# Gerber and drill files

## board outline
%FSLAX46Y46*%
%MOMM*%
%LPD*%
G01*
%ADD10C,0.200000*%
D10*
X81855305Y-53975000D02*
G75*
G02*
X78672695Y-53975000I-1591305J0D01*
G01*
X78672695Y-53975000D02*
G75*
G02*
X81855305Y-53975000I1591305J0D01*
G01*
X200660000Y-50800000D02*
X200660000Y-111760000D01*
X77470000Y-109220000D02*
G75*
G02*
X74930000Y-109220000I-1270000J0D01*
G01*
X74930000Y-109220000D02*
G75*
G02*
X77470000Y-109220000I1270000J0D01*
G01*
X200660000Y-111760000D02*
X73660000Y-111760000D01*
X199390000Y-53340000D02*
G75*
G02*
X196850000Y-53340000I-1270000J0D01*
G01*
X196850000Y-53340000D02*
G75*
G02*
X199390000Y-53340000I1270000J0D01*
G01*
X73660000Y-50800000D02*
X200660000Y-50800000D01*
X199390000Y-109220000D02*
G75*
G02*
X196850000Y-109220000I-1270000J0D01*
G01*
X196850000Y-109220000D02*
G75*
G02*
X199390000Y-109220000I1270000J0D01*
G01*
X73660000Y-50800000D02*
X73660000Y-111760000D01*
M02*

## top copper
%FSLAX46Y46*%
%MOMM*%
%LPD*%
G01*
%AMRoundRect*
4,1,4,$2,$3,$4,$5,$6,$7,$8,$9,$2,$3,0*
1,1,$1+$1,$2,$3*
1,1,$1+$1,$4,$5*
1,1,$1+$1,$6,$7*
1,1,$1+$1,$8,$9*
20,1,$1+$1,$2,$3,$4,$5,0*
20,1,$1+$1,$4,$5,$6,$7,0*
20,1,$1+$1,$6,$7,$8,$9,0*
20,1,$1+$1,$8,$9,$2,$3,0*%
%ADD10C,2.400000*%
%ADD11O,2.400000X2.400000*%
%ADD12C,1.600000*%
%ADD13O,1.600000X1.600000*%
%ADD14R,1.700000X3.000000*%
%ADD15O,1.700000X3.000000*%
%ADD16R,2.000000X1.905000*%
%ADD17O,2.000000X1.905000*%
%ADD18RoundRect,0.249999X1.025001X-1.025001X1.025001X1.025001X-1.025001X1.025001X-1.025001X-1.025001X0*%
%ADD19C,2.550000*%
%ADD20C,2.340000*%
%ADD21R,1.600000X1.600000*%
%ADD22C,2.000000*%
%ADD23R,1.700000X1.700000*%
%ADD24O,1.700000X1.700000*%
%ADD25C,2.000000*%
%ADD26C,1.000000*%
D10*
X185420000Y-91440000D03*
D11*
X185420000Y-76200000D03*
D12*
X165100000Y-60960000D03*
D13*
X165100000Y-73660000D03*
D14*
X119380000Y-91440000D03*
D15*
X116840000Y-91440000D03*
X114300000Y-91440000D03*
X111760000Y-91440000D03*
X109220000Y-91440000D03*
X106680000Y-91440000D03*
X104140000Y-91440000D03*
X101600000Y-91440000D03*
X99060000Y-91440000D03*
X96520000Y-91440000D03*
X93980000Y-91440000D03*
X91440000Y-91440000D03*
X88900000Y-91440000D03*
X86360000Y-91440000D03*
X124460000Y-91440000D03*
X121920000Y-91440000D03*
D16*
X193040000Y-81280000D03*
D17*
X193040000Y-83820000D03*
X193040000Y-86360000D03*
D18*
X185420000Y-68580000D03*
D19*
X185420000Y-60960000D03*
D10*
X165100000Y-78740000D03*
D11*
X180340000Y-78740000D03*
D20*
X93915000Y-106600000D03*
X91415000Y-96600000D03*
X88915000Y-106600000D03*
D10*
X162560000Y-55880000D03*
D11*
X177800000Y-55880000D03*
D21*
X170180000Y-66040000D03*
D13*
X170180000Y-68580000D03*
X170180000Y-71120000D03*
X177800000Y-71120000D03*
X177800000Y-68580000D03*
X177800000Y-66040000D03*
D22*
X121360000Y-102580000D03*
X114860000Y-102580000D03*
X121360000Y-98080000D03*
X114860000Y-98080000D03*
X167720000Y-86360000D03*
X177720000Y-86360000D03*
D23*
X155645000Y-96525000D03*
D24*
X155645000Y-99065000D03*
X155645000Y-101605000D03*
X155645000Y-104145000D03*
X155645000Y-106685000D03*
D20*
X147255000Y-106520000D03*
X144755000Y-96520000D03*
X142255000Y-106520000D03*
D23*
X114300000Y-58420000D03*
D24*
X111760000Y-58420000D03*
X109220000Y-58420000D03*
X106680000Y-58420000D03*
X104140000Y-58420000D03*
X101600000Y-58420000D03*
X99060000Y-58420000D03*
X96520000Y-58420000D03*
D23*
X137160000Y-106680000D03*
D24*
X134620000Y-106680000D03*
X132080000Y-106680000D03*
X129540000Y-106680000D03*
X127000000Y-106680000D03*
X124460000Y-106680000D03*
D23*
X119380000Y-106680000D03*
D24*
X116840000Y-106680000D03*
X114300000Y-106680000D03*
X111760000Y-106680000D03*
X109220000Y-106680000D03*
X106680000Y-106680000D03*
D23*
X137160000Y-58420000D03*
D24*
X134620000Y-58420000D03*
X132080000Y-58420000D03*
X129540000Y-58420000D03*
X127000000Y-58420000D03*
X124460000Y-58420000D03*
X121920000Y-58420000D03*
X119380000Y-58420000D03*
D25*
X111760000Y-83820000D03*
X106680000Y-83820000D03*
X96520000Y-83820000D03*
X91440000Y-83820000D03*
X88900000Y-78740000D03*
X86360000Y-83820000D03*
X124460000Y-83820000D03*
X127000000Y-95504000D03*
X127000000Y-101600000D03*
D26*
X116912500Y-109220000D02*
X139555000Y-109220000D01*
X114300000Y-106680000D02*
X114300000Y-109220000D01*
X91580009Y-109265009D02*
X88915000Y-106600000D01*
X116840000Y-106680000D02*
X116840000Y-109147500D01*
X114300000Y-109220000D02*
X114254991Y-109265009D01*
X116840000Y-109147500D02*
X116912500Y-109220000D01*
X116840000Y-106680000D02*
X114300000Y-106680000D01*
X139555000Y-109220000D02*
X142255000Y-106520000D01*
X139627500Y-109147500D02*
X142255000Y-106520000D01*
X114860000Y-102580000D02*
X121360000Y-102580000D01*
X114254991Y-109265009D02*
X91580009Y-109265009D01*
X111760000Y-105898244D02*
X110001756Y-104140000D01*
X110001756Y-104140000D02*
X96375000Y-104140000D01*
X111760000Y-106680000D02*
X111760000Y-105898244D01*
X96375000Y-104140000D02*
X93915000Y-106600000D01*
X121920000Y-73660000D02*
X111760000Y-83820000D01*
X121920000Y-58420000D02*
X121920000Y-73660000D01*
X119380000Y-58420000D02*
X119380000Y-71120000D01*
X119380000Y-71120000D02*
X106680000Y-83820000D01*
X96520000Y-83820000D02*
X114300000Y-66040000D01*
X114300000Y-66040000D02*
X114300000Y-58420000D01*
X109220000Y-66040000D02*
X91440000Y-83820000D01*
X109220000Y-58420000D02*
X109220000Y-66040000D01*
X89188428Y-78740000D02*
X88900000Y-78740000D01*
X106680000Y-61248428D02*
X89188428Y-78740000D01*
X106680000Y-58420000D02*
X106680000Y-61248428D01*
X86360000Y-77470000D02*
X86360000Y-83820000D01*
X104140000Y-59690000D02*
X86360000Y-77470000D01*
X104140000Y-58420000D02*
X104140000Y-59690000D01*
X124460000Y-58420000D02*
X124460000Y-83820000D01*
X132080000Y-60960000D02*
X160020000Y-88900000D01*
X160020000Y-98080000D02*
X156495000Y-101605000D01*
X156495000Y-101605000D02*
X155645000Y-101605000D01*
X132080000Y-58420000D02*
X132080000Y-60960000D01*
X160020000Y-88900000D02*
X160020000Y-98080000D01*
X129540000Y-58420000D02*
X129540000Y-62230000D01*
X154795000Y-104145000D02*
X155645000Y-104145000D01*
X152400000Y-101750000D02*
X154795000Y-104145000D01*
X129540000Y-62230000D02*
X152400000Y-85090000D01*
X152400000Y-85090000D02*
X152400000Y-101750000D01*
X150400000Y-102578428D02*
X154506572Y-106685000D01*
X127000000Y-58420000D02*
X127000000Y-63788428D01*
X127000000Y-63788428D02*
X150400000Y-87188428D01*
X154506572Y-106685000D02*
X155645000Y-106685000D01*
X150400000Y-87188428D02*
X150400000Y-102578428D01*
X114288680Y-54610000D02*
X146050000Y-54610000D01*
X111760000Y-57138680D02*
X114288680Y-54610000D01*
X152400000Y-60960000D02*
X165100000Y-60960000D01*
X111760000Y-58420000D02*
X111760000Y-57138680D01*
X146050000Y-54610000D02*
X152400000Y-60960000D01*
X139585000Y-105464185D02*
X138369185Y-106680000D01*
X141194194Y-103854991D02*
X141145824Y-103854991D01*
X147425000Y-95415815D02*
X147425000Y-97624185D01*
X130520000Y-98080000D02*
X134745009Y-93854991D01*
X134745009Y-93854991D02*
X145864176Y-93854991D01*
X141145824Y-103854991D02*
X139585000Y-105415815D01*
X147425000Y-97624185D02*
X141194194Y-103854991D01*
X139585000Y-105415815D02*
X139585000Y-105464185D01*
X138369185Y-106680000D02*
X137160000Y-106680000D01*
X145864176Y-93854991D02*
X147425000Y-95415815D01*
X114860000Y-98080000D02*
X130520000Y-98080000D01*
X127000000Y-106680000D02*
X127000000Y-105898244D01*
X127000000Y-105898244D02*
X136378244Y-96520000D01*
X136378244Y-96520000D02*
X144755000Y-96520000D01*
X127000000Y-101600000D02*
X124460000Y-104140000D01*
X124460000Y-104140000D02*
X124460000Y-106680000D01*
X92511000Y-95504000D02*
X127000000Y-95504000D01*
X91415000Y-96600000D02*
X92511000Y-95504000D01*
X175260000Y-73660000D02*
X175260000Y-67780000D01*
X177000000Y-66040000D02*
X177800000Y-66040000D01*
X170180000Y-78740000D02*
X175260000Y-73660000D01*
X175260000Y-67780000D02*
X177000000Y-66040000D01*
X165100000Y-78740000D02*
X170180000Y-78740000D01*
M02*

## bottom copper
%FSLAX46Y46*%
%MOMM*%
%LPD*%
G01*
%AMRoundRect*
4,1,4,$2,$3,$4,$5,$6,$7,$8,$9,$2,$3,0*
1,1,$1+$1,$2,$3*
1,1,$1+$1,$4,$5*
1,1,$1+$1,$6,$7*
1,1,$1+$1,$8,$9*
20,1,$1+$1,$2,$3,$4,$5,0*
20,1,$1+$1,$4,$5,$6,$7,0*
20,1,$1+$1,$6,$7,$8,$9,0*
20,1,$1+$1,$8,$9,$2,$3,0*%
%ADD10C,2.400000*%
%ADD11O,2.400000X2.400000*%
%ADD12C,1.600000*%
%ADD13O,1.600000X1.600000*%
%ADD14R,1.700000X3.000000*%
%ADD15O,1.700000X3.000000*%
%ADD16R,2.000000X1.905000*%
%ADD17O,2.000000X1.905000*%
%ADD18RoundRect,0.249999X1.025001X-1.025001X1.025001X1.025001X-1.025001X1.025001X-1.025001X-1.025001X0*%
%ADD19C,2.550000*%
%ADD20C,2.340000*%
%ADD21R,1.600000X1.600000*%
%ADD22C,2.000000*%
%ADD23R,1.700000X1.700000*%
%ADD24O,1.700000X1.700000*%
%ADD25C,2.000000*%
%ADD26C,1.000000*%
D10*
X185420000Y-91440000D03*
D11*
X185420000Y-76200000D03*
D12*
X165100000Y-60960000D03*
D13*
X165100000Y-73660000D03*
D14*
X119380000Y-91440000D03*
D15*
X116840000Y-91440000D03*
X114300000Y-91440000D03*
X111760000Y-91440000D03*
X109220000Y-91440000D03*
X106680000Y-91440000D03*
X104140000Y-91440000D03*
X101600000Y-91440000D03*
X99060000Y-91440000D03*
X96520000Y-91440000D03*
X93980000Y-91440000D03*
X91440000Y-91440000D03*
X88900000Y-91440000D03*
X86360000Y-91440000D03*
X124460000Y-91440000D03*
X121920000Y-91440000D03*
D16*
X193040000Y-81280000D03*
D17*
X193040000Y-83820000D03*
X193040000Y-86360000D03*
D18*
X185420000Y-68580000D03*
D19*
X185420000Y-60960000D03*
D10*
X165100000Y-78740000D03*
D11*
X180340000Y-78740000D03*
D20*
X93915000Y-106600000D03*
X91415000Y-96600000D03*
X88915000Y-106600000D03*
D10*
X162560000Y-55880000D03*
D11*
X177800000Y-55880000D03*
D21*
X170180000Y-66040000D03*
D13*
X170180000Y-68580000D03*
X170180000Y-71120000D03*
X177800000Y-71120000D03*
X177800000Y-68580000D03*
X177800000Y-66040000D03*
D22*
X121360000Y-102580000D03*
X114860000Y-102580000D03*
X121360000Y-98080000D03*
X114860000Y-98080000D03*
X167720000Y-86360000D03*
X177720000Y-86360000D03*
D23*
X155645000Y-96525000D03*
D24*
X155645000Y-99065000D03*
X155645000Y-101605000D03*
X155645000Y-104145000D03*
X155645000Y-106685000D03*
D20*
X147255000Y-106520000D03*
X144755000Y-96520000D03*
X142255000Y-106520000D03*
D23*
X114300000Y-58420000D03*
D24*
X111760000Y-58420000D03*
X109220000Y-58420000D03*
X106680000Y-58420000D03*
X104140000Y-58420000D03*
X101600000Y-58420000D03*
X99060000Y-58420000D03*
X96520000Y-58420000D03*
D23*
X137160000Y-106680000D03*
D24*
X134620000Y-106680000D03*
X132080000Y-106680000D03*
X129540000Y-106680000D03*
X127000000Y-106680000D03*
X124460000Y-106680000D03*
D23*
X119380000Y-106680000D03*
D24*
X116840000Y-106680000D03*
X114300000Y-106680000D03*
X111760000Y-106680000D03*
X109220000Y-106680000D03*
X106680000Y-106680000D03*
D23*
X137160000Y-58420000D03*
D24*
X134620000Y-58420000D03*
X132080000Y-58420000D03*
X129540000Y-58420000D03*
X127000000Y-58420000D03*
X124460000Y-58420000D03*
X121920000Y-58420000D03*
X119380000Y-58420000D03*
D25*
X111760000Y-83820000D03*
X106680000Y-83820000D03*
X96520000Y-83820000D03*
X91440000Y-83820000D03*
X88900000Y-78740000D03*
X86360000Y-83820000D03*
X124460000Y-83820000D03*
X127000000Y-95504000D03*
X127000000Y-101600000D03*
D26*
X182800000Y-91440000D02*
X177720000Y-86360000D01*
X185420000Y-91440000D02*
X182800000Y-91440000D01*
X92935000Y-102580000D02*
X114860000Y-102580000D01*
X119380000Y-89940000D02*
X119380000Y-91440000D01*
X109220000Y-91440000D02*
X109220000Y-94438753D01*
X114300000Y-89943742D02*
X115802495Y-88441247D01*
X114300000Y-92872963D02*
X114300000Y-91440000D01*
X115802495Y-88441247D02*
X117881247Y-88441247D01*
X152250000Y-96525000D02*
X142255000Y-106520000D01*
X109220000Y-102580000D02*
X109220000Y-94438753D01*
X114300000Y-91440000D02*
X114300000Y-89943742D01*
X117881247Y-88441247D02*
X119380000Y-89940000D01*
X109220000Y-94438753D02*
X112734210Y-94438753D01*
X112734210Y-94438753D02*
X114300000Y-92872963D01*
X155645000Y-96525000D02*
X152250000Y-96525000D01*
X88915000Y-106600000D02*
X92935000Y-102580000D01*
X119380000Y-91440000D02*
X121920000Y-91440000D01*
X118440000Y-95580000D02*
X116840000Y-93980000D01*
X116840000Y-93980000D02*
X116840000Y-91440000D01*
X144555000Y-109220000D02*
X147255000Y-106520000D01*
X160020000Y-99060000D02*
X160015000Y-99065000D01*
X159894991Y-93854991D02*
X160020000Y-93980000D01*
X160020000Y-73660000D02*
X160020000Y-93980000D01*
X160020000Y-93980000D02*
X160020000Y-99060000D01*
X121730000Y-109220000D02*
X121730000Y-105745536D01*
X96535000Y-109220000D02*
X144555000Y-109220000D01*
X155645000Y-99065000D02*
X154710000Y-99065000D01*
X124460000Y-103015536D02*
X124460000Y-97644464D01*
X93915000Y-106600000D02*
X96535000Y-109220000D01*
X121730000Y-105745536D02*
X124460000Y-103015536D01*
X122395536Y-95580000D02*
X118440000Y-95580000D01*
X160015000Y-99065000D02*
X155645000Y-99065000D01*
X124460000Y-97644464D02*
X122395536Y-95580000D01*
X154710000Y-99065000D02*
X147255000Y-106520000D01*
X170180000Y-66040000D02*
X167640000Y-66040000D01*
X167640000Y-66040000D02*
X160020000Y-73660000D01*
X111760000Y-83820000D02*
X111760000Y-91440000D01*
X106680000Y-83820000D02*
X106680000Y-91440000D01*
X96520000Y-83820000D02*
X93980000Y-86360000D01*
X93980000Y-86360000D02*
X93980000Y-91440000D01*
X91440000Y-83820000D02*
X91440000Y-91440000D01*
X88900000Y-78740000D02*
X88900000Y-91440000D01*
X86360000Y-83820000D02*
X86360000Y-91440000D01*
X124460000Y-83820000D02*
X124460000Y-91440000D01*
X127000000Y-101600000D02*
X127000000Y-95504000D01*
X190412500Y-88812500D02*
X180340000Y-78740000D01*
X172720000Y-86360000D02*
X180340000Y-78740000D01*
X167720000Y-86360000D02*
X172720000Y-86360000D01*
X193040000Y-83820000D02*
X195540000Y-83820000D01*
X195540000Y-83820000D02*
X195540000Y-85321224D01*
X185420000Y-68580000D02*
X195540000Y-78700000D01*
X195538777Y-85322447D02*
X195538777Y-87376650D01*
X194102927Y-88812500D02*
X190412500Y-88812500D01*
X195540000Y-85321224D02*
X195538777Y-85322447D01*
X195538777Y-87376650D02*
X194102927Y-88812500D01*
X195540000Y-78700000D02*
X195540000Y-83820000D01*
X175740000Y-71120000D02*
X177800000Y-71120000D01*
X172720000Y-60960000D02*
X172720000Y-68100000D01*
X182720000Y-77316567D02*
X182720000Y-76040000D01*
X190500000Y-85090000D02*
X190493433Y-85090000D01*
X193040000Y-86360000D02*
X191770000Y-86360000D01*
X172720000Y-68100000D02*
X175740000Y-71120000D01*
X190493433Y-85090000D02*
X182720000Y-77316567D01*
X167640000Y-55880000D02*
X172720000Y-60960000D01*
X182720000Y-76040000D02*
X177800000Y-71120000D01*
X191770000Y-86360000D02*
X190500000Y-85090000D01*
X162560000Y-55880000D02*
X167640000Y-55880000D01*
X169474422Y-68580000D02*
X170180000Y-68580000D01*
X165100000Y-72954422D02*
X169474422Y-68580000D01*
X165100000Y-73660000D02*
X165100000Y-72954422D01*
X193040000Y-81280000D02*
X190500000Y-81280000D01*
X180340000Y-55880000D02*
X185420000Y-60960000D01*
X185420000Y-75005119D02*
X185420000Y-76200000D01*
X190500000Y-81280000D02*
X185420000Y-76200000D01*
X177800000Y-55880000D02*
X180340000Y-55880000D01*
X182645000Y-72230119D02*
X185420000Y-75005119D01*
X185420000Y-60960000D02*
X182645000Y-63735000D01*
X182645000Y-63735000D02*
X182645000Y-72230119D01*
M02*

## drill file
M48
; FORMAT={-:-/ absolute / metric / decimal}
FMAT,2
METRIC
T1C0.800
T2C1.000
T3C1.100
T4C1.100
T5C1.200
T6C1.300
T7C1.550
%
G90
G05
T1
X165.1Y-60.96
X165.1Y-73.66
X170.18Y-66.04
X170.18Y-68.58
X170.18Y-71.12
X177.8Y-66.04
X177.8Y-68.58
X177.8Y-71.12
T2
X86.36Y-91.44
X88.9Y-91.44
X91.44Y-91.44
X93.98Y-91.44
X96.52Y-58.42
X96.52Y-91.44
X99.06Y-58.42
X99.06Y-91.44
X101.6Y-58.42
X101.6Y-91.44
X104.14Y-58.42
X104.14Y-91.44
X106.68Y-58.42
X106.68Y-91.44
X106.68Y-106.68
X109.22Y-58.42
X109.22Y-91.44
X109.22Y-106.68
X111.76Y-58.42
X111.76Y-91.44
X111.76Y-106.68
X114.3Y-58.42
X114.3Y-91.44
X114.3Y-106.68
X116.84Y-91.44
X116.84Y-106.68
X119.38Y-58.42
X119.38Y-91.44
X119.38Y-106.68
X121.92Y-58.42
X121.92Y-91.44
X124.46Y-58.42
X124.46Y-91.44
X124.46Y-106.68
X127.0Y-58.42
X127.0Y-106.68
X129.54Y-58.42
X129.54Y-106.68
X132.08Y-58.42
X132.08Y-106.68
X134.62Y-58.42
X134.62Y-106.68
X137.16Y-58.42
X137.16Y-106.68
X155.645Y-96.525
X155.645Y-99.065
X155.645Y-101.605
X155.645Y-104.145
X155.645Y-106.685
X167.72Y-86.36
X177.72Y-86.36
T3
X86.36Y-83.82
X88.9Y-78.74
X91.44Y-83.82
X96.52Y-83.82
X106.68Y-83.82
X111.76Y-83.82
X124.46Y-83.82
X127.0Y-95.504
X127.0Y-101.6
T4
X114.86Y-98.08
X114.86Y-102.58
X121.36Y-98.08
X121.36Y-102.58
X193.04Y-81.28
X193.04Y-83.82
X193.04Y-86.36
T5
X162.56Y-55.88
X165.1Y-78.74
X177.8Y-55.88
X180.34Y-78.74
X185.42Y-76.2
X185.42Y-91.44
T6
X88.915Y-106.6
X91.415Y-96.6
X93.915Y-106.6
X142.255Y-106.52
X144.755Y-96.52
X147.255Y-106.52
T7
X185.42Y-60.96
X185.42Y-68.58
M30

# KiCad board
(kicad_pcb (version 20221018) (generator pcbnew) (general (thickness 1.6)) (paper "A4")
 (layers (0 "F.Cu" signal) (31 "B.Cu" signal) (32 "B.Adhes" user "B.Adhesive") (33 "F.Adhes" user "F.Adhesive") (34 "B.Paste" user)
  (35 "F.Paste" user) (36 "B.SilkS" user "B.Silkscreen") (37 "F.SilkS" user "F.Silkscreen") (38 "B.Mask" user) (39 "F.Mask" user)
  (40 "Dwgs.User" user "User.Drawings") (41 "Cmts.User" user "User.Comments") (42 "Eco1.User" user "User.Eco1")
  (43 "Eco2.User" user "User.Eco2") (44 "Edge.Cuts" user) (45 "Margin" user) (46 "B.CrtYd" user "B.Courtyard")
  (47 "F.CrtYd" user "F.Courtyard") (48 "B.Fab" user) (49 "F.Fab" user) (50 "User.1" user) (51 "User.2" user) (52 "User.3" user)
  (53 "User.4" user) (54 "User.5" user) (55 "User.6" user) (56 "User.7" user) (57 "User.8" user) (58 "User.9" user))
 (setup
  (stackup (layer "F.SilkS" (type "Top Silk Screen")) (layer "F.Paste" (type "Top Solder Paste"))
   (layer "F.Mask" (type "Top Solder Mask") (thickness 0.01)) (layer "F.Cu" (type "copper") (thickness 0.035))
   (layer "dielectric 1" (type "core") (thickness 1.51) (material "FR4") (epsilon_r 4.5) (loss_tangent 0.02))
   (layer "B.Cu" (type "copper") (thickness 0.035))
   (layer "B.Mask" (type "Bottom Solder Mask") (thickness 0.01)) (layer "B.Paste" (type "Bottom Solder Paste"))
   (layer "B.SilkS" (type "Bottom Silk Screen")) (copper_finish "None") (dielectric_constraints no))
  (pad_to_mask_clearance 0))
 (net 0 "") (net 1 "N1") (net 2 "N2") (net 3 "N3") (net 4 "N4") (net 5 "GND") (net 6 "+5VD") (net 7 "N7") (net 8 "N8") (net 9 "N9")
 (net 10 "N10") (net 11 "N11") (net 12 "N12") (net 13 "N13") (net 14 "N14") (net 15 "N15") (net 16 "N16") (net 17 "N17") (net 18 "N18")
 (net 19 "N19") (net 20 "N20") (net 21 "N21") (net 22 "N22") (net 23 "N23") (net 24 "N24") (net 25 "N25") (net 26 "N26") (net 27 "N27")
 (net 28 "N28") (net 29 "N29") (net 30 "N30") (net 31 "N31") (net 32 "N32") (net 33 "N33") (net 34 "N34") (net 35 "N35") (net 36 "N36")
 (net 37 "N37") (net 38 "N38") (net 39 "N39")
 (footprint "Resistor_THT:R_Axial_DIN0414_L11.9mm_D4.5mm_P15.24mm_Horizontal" (layer "F.Cu") (at 185.42 91.44 90)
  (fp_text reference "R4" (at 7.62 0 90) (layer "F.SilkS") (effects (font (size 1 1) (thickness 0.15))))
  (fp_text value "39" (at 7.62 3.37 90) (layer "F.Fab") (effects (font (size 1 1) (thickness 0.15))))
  (pad "1" thru_hole circle (at 0 0 90) (size 2.4 2.4) (drill 1.2) (layers "*.Cu" "*.Mask") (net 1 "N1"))
  (pad "2" thru_hole oval (at 15.24 0 90) (size 2.4 2.4) (drill 1.2) (layers "*.Cu" "*.Mask") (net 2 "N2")))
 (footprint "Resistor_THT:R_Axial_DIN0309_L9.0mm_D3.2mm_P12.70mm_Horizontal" (layer "F.Cu") (at 165.1 60.96 -90)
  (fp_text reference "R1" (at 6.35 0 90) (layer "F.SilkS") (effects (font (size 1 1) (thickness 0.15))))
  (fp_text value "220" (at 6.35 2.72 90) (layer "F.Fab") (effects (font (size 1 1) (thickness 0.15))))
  (pad "1" thru_hole circle (at 0 0 270) (size 1.6 1.6) (drill 0.8) (layers "*.Cu" "*.Mask") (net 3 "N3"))
  (pad "2" thru_hole oval (at 12.7 0 270) (size 1.6 1.6) (drill 0.8) (layers "*.Cu" "*.Mask") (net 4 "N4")))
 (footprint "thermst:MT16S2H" (layer "F.Cu") (at 86.36 91.44)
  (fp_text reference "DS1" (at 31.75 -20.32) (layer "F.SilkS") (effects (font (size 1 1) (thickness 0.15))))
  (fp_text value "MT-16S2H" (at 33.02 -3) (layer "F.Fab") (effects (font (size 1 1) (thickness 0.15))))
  (pad "1" thru_hole rect (at 33.02 0 180) (size 1.7 3) (drill oval 1) (layers "*.Cu" "*.Mask") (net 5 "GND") (thermal_bridge_angle 45))
  (pad "2" thru_hole oval (at 30.48 0 180) (size 1.7 3) (drill 1) (layers "*.Cu" "*.Mask") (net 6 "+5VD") (thermal_bridge_angle 45))
  (pad "3" thru_hole oval (at 27.94 0 180) (size 1.7 3) (drill 1) (layers "*.Cu" "*.Mask") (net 5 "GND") (thermal_bridge_angle 45))
  (pad "4" thru_hole oval (at 25.4 0 180) (size 1.7 3) (drill 1) (layers "*.Cu" "*.Mask") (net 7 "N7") (thermal_bridge_angle 45))
  (pad "5" thru_hole oval (at 22.86 0 180) (size 1.7 3) (drill 1) (layers "*.Cu" "*.Mask") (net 5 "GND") (thermal_bridge_angle 45))
  (pad "6" thru_hole oval (at 20.32 0 180) (size 1.7 3) (drill 1) (layers "*.Cu" "*.Mask") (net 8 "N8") (thermal_bridge_angle 45))
  (pad "7" thru_hole oval (at 17.78 0 180) (size 1.7 3) (drill 1) (layers "*.Cu" "*.Mask") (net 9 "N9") (thermal_bridge_angle 45))
  (pad "8" thru_hole oval (at 15.24 0 180) (size 1.7 3) (drill 1) (layers "*.Cu" "*.Mask") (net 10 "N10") (thermal_bridge_angle 45))
  (pad "9" thru_hole oval (at 12.7 0 180) (size 1.7 3) (drill 1) (layers "*.Cu" "*.Mask") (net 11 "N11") (thermal_bridge_angle 45))
  (pad "10" thru_hole oval (at 10.16 0 180) (size 1.7 3) (drill 1) (layers "*.Cu" "*.Mask") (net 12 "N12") (thermal_bridge_angle 45))
  (pad "11" thru_hole oval (at 7.62 0 180) (size 1.7 3) (drill 1) (layers "*.Cu" "*.Mask") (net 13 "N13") (thermal_bridge_angle 45))
  (pad "12" thru_hole oval (at 5.08 0 180) (size 1.7 3) (drill 1) (layers "*.Cu" "*.Mask") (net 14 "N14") (thermal_bridge_angle 45))
  (pad "13" thru_hole oval (at 2.54 0 180) (size 1.7 3) (drill 1) (layers "*.Cu" "*.Mask") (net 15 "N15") (thermal_bridge_angle 45))
  (pad "14" thru_hole oval (at 0 0 180) (size 1.7 3) (drill 1) (layers "*.Cu" "*.Mask") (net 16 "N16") (thermal_bridge_angle 45))
  (pad "15" thru_hole oval (at 38.1 0 180) (size 1.7 3) (drill 1) (layers "*.Cu" "*.Mask") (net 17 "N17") (thermal_bridge_angle 45))
  (pad "16" thru_hole oval (at 35.56 0 180) (size 1.7 3) (drill 1) (layers "*.Cu" "*.Mask") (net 5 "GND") (thermal_bridge_angle 45)))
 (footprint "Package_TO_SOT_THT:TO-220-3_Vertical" (layer "F.Cu") (at 193.04 81.28 -90)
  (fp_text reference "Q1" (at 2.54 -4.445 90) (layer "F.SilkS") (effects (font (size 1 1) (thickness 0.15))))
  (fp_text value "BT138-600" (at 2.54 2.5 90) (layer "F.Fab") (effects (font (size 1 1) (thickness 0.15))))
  (pad "1" thru_hole rect (at 0 0 270) (size 1.905 2) (drill 1.1) (layers "*.Cu" "*.Mask") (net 2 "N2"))
  (pad "2" thru_hole oval (at 2.54 0 270) (size 1.905 2) (drill 1.1) (layers "*.Cu" "*.Mask") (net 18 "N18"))
  (pad "3" thru_hole oval (at 5.08 0 270) (size 1.905 2) (drill 1.1) (layers "*.Cu" "*.Mask") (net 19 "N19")))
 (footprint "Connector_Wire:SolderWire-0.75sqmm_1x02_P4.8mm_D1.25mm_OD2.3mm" (layer "F.Cu") (at 185.42 68.58 90)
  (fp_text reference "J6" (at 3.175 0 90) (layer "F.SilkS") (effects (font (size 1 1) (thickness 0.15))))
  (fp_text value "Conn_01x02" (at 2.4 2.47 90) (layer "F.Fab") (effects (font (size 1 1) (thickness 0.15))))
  (pad "1" thru_hole roundrect (at 0 0 90) (size 2.55 2.55) (drill 1.55) (layers "*.Cu" "*.Mask") (roundrect_rratio 0.098039) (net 18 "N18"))
  (pad "2" thru_hole circle (at 7.62 0 90) (size 2.55 2.55) (drill 1.55) (layers "*.Cu" "*.Mask") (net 2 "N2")))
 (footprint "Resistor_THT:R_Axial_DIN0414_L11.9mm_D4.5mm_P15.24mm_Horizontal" (layer "F.Cu") (at 165.1 78.74)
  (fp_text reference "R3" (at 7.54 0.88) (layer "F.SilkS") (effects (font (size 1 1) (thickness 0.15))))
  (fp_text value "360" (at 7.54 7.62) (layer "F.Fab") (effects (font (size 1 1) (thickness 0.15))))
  (pad "1" thru_hole circle (at 0 0) (size 2.4 2.4) (drill 1.2) (layers "*.Cu" "*.Mask") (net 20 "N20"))
  (pad "2" thru_hole oval (at 15.24 0) (size 2.4 2.4) (drill 1.2) (layers "*.Cu" "*.Mask") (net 18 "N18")))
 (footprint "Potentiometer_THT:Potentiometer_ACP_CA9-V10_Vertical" (layer "F.Cu") (at 93.915 106.6 90)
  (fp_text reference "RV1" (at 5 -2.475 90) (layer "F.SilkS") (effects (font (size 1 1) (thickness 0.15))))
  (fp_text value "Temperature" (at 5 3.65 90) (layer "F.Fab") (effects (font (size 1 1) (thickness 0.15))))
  (pad "1" thru_hole circle (at 0 0 90) (size 2.34 2.34) (drill 1.3) (layers "*.Cu" "*.Mask") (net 6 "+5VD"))
  (pad "2" thru_hole circle (at 10 -2.5 90) (size 2.34 2.34) (drill 1.3) (layers "*.Cu" "*.Mask") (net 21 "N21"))
  (pad "3" thru_hole circle (at 0 -5 90) (size 2.34 2.34) (drill 1.3) (layers "*.Cu" "*.Mask") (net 5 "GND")))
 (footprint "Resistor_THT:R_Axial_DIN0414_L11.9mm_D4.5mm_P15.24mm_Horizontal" (layer "F.Cu") (at 162.56 55.88)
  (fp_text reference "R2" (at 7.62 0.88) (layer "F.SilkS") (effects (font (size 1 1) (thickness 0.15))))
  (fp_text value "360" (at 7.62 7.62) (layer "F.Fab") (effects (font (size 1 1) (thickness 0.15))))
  (pad "1" thru_hole circle (at 0 0) (size 2.4 2.4) (drill 1.2) (layers "*.Cu" "*.Mask") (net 19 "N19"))
  (pad "2" thru_hole oval (at 15.24 0) (size 2.4 2.4) (drill 1.2) (layers "*.Cu" "*.Mask") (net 2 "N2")))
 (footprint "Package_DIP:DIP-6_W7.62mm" (layer "F.Cu") (at 170.18 66.04)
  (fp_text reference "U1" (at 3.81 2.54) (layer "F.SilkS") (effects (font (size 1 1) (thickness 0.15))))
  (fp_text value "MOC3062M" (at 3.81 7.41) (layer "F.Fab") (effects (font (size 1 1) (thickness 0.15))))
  (pad "1" thru_hole rect (at 0 0) (size 1.6 1.6) (drill 0.8) (layers "*.Cu" "*.Mask") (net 6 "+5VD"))
  (pad "2" thru_hole oval (at 0 2.54) (size 1.6 1.6) (drill 0.8) (layers "*.Cu" "*.Mask") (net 4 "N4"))
  (pad "3" thru_hole oval (at 0 5.08) (size 1.6 1.6) (drill 0.8) (layers "*.Cu" "*.Mask") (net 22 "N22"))
  (pad "4" thru_hole oval (at 7.62 5.08) (size 1.6 1.6) (drill 0.8) (layers "*.Cu" "*.Mask") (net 19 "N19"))
  (pad "5" thru_hole oval (at 7.62 2.54) (size 1.6 1.6) (drill 0.8) (layers "*.Cu" "*.Mask") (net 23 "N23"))
  (pad "6" thru_hole oval (at 7.62 0) (size 1.6 1.6) (drill 0.8) (layers "*.Cu" "*.Mask") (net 20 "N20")))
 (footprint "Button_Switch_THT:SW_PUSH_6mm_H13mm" (layer "F.Cu") (at 121.36 102.58 180)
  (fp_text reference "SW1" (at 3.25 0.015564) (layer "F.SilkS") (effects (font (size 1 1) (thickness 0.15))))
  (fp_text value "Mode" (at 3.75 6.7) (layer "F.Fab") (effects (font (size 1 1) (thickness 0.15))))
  (pad "1" thru_hole circle (at 0 0 270) (size 2 2) (drill 1.1) (layers "*.Cu" "*.Mask") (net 5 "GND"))
  (pad "1" thru_hole circle (at 6.5 0 270) (size 2 2) (drill 1.1) (layers "*.Cu" "*.Mask") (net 5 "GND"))
  (pad "2" thru_hole circle (at 0 4.5 270) (size 2 2) (drill 1.1) (layers "*.Cu" "*.Mask") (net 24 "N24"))
  (pad "2" thru_hole circle (at 6.5 4.5 270) (size 2 2) (drill 1.1) (layers "*.Cu" "*.Mask") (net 24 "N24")))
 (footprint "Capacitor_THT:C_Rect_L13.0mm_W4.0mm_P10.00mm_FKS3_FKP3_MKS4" (layer "F.Cu") (at 167.72 86.36)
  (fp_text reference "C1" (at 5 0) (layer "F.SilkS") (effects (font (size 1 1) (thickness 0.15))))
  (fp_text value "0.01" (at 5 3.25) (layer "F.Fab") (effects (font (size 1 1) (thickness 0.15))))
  (pad "1" thru_hole circle (at 0 0) (size 2 2) (drill 1) (layers "*.Cu" "*.Mask") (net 18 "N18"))
  (pad "2" thru_hole circle (at 10 0) (size 2 2) (drill 1) (layers "*.Cu" "*.Mask") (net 1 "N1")))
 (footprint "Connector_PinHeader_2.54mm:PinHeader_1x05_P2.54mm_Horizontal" (layer "F.Cu") (at 155.645 96.525)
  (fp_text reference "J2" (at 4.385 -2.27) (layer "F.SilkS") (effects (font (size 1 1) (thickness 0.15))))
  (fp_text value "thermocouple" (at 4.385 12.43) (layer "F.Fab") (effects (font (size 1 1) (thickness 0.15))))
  (pad "1" thru_hole rect (at 0 0) (size 1.7 1.7) (drill 1) (layers "*.Cu" "*.Mask") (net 5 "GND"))
  (pad "2" thru_hole oval (at 0 2.54) (size 1.7 1.7) (drill 1) (layers "*.Cu" "*.Mask") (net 6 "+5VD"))
  (pad "3" thru_hole oval (at 0 5.08) (size 1.7 1.7) (drill 1) (layers "*.Cu" "*.Mask") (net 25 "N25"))
  (pad "4" thru_hole oval (at 0 7.62) (size 1.7 1.7) (drill 1) (layers "*.Cu" "*.Mask") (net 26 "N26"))
  (pad "5" thru_hole oval (at 0 10.16) (size 1.7 1.7) (drill 1) (layers "*.Cu" "*.Mask") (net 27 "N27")))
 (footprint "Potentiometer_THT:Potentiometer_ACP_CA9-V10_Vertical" (layer "F.Cu") (at 147.255 106.52 90)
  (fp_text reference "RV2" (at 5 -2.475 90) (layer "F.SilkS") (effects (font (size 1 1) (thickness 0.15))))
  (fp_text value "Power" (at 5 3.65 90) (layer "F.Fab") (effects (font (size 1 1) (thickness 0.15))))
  (pad "1" thru_hole circle (at 0 0 90) (size 2.34 2.34) (drill 1.3) (layers "*.Cu" "*.Mask") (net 6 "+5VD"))
  (pad "2" thru_hole circle (at 10 -2.5 90) (size 2.34 2.34) (drill 1.3) (layers "*.Cu" "*.Mask") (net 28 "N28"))
  (pad "3" thru_hole circle (at 0 -5 90) (size 2.34 2.34) (drill 1.3) (layers "*.Cu" "*.Mask") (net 5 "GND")))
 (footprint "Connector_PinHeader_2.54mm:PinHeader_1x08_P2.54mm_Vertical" (layer "B.Cu") (at 114.3 58.42 90)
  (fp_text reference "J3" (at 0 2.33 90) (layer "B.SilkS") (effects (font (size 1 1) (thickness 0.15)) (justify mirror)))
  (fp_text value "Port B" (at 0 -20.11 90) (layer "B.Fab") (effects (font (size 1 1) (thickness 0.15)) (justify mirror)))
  (pad "1" thru_hole rect (at 0 0 90) (size 1.7 1.7) (drill 1) (layers "*.Cu" "*.Mask") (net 13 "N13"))
  (pad "2" thru_hole oval (at 0 -2.54 90) (size 1.7 1.7) (drill 1) (layers "*.Cu" "*.Mask") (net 3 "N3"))
  (pad "3" thru_hole oval (at 0 -5.08 90) (size 1.7 1.7) (drill 1) (layers "*.Cu" "*.Mask") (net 14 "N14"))
  (pad "4" thru_hole oval (at 0 -7.62 90) (size 1.7 1.7) (drill 1) (layers "*.Cu" "*.Mask") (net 15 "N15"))
  (pad "5" thru_hole oval (at 0 -10.16 90) (size 1.7 1.7) (drill 1) (layers "*.Cu" "*.Mask") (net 16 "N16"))
  (pad "6" thru_hole oval (at 0 -12.7 90) (size 1.7 1.7) (drill 1) (layers "*.Cu" "*.Mask") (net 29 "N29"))
  (pad "7" thru_hole oval (at 0 -15.24 90) (size 1.7 1.7) (drill 1) (layers "*.Cu" "*.Mask") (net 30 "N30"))
  (pad "8" thru_hole oval (at 0 -17.78 90) (size 1.7 1.7) (drill 1) (layers "*.Cu" "*.Mask") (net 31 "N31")))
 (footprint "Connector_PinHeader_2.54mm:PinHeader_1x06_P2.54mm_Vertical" (layer "B.Cu") (at 137.16 106.68 90)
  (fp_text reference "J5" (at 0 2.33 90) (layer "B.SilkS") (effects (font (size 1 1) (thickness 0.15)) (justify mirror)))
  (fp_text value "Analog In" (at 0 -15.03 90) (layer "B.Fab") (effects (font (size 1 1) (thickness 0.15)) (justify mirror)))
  (pad "1" thru_hole rect (at 0 0 90) (size 1.7 1.7) (drill 1) (layers "*.Cu" "*.Mask") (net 24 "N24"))
  (pad "2" thru_hole oval (at 0 -2.54 90) (size 1.7 1.7) (drill 1) (layers "*.Cu" "*.Mask") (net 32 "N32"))
  (pad "3" thru_hole oval (at 0 -5.08 90) (size 1.7 1.7) (drill 1) (layers "*.Cu" "*.Mask") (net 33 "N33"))
  (pad "4" thru_hole oval (at 0 -7.62 90) (size 1.7 1.7) (drill 1) (layers "*.Cu" "*.Mask") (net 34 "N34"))
  (pad "5" thru_hole oval (at 0 -10.16 90) (size 1.7 1.7) (drill 1) (layers "*.Cu" "*.Mask") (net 28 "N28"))
  (pad "6" thru_hole oval (at 0 -12.7 90) (size 1.7 1.7) (drill 1) (layers "*.Cu" "*.Mask") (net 21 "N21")))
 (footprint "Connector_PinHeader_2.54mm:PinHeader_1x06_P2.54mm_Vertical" (layer "B.Cu") (at 119.38 106.68 90)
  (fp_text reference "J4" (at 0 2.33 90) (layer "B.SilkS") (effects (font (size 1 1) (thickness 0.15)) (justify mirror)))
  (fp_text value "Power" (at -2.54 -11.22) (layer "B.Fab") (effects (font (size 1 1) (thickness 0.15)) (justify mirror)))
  (pad "1" thru_hole rect (at 0 0 90) (size 1.7 1.7) (drill 1) (layers "*.Cu" "*.Mask") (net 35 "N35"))
  (pad "2" thru_hole oval (at 0 -2.54 90) (size 1.7 1.7) (drill 1) (layers "*.Cu" "*.Mask") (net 5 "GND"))
  (pad "3" thru_hole oval (at 0 -5.08 90) (size 1.7 1.7) (drill 1) (layers "*.Cu" "*.Mask") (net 5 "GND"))
  (pad "4" thru_hole oval (at 0 -7.62 90) (size 1.7 1.7) (drill 1) (layers "*.Cu" "*.Mask") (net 6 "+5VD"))
  (pad "5" thru_hole oval (at 0 -10.16 90) (size 1.7 1.7) (drill 1) (layers "*.Cu" "*.Mask") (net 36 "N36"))
  (pad "6" thru_hole oval (at 0 -12.7 90) (size 1.7 1.7) (drill 1) (layers "*.Cu" "*.Mask") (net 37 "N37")))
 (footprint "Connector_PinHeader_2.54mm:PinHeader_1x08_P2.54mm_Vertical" (layer "B.Cu") (at 137.16 58.42 90)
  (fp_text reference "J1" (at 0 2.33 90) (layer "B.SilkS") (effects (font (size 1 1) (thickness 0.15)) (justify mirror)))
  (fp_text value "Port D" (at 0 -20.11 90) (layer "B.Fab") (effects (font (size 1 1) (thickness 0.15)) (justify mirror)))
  (pad "1" thru_hole rect (at 0 0 90) (size 1.7 1.7) (drill 1) (layers "*.Cu" "*.Mask") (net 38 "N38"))
  (pad "2" thru_hole oval (at 0 -2.54 90) (size 1.7 1.7) (drill 1) (layers "*.Cu" "*.Mask") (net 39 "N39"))
  (pad "3" thru_hole oval (at 0 -5.08 90) (size 1.7 1.7) (drill 1) (layers "*.Cu" "*.Mask") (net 25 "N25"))
  (pad "4" thru_hole oval (at 0 -7.62 90) (size 1.7 1.7) (drill 1) (layers "*.Cu" "*.Mask") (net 26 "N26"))
  (pad "5" thru_hole oval (at 0 -10.16 90) (size 1.7 1.7) (drill 1) (layers "*.Cu" "*.Mask") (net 27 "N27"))
  (pad "6" thru_hole oval (at 0 -12.7 90) (size 1.7 1.7) (drill 1) (layers "*.Cu" "*.Mask") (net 17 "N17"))
  (pad "7" thru_hole oval (at 0 -15.24 90) (size 1.7 1.7) (drill 1) (layers "*.Cu" "*.Mask") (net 7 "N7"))
  (pad "8" thru_hole oval (at 0 -17.78 90) (size 1.7 1.7) (drill 1) (layers "*.Cu" "*.Mask") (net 8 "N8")))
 (gr_circle (center 80.264 53.975) (end 78.867 53.213) (stroke (width 0.2) (type default)) (fill none) (layer "Edge.Cuts"))
 (gr_line (start 200.66 50.8) (end 200.66 111.76) (stroke (width 0.2) (type default)) (layer "Edge.Cuts"))
 (gr_circle (center 76.2 109.22) (end 77.47 109.22) (stroke (width 0.2) (type default)) (fill none) (layer "Edge.Cuts"))
 (gr_line (start 200.66 111.76) (end 73.66 111.76) (stroke (width 0.2) (type default)) (layer "Edge.Cuts"))
 (gr_circle (center 198.12 53.34) (end 198.12 52.07) (stroke (width 0.2) (type default)) (fill none) (layer "Edge.Cuts"))
 (gr_line (start 73.66 50.8) (end 200.66 50.8) (stroke (width 0.2) (type default)) (layer "Edge.Cuts"))
 (gr_circle (center 198.12 109.22) (end 198.12 107.95) (stroke (width 0.2) (type default)) (fill none) (layer "Edge.Cuts"))
 (gr_line (start 73.66 50.8) (end 73.66 111.76) (stroke (width 0.2) (type default)) (layer "Edge.Cuts"))
 (segment (start 182.8 91.44) (end 177.72 86.36) (width 1) (layer "B.Cu") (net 1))
 (segment (start 185.42 91.44) (end 182.8 91.44) (width 1) (layer "B.Cu") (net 1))
 (segment (start 116.9125 109.22) (end 139.555 109.22) (width 1) (layer "F.Cu") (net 5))
 (segment (start 114.3 106.68) (end 114.3 109.22) (width 1) (layer "F.Cu") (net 5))
 (segment (start 91.580009 109.265009) (end 88.915 106.6) (width 1) (layer "F.Cu") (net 5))
 (segment (start 116.84 106.68) (end 116.84 109.1475) (width 1) (layer "F.Cu") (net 5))
 (segment (start 114.3 109.22) (end 114.254991 109.265009) (width 1) (layer "F.Cu") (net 5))
 (segment (start 116.84 109.1475) (end 116.9125 109.22) (width 1) (layer "F.Cu") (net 5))
 (segment (start 116.84 106.68) (end 114.3 106.68) (width 1) (layer "F.Cu") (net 5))
 (segment (start 139.555 109.22) (end 142.255 106.52) (width 1) (layer "F.Cu") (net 5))
 (segment (start 139.6275 109.1475) (end 142.255 106.52) (width 1) (layer "F.Cu") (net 5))
 (segment (start 114.86 102.58) (end 121.36 102.58) (width 1) (layer "F.Cu") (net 5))
 (segment (start 114.254991 109.265009) (end 91.580009 109.265009) (width 1) (layer "F.Cu") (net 5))
 (segment (start 92.935 102.58) (end 114.86 102.58) (width 1) (layer "B.Cu") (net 5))
 (segment (start 119.38 89.94) (end 119.38 91.44) (width 1) (layer "B.Cu") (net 5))
 (segment (start 109.22 91.44) (end 109.22 94.438753) (width 1) (layer "B.Cu") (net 5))
 (segment (start 114.3 89.943742) (end 115.802495 88.441247) (width 1) (layer "B.Cu") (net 5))
 (segment (start 114.3 92.872963) (end 114.3 91.44) (width 1) (layer "B.Cu") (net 5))
 (segment (start 115.802495 88.441247) (end 117.881247 88.441247) (width 1) (layer "B.Cu") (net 5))
 (segment (start 152.25 96.525) (end 142.255 106.52) (width 1) (layer "B.Cu") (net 5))
 (segment (start 109.22 102.58) (end 109.22 94.438753) (width 1) (layer "B.Cu") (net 5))
 (segment (start 114.3 91.44) (end 114.3 89.943742) (width 1) (layer "B.Cu") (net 5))
 (segment (start 117.881247 88.441247) (end 119.38 89.94) (width 1) (layer "B.Cu") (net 5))
 (segment (start 109.22 94.438753) (end 112.73421 94.438753) (width 1) (layer "B.Cu") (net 5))
 (segment (start 112.73421 94.438753) (end 114.3 92.872963) (width 1) (layer "B.Cu") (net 5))
 (segment (start 155.645 96.525) (end 152.25 96.525) (width 1) (layer "B.Cu") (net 5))
 (segment (start 88.915 106.6) (end 92.935 102.58) (width 1) (layer "B.Cu") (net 5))
 (segment (start 119.38 91.44) (end 121.92 91.44) (width 1) (layer "B.Cu") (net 5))
 (segment (start 111.76 105.898244) (end 110.001756 104.14) (width 1) (layer "F.Cu") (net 6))
 (segment (start 110.001756 104.14) (end 96.375 104.14) (width 1) (layer "F.Cu") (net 6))
 (segment (start 111.76 106.68) (end 111.76 105.898244) (width 1) (layer "F.Cu") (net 6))
 (segment (start 96.375 104.14) (end 93.915 106.6) (width 1) (layer "F.Cu") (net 6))
 (segment (start 118.44 95.58) (end 116.84 93.98) (width 1) (layer "B.Cu") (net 6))
 (segment (start 116.84 93.98) (end 116.84 91.44) (width 1) (layer "B.Cu") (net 6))
 (segment (start 144.555 109.22) (end 147.255 106.52) (width 1) (layer "B.Cu") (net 6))
 (segment (start 160.02 99.06) (end 160.015 99.065) (width 1) (layer "B.Cu") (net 6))
 (segment (start 159.894991 93.854991) (end 160.02 93.98) (width 1) (layer "B.Cu") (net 6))
 (segment (start 160.02 73.66) (end 160.02 93.98) (width 1) (layer "B.Cu") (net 6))
 (segment (start 160.02 93.98) (end 160.02 99.06) (width 1) (layer "B.Cu") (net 6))
 (segment (start 121.73 109.22) (end 121.73 105.745536) (width 1) (layer "B.Cu") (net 6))
 (segment (start 96.535 109.22) (end 144.555 109.22) (width 1) (layer "B.Cu") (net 6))
 (segment (start 155.645 99.065) (end 154.71 99.065) (width 1) (layer "B.Cu") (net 6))
 (segment (start 124.46 103.015536) (end 124.46 97.644464) (width 1) (layer "B.Cu") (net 6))
 (segment (start 93.915 106.6) (end 96.535 109.22) (width 1) (layer "B.Cu") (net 6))
 (segment (start 121.73 105.745536) (end 124.46 103.015536) (width 1) (layer "B.Cu") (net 6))
 (segment (start 122.395536 95.58) (end 118.44 95.58) (width 1) (layer "B.Cu") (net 6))
 (segment (start 160.015 99.065) (end 155.645 99.065) (width 1) (layer "B.Cu") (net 6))
 (segment (start 124.46 97.644464) (end 122.395536 95.58) (width 1) (layer "B.Cu") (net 6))
 (segment (start 154.71 99.065) (end 147.255 106.52) (width 1) (layer "B.Cu") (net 6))
 (segment (start 170.18 66.04) (end 167.64 66.04) (width 1) (layer "B.Cu") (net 6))
 (segment (start 167.64 66.04) (end 160.02 73.66) (width 1) (layer "B.Cu") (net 6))
 (segment (start 121.92 73.66) (end 111.76 83.82) (width 1) (layer "F.Cu") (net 7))
 (segment (start 121.92 58.42) (end 121.92 73.66) (width 1) (layer "F.Cu") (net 7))
 (via (at 111.76 83.82) (size 2) (drill 1.1) (layers "F.Cu" "B.Cu") (free) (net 7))
 (segment (start 111.76 83.82) (end 111.76 91.44) (width 1) (layer "B.Cu") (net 7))
 (segment (start 119.38 58.42) (end 119.38 71.12) (width 1) (layer "F.Cu") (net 8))
 (segment (start 119.38 71.12) (end 106.68 83.82) (width 1) (layer "F.Cu") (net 8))
 (via (at 106.68 83.82) (size 2) (drill 1.1) (layers "F.Cu" "B.Cu") (free) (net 8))
 (segment (start 106.68 83.82) (end 106.68 91.44) (width 1) (layer "B.Cu") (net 8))
 (segment (start 96.52 83.82) (end 114.3 66.04) (width 1) (layer "F.Cu") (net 13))
 (segment (start 114.3 66.04) (end 114.3 58.42) (width 1) (layer "F.Cu") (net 13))
 (via (at 96.52 83.82) (size 2) (drill 1.1) (layers "F.Cu" "B.Cu") (free) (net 13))
 (segment (start 96.52 83.82) (end 93.98 86.36) (width 1) (layer "B.Cu") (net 13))
 (segment (start 93.98 86.36) (end 93.98 91.44) (width 1) (layer "B.Cu") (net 13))
 (segment (start 109.22 66.04) (end 91.44 83.82) (width 1) (layer "F.Cu") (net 14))
 (segment (start 109.22 58.42) (end 109.22 66.04) (width 1) (layer "F.Cu") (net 14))
 (via (at 91.44 83.82) (size 2) (drill 1.1) (layers "F.Cu" "B.Cu") (free) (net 14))
 (segment (start 91.44 83.82) (end 91.44 91.44) (width 1) (layer "B.Cu") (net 14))
 (segment (start 89.188428 78.74) (end 88.9 78.74) (width 1) (layer "F.Cu") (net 15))
 (segment (start 106.68 61.248428) (end 89.188428 78.74) (width 1) (layer "F.Cu") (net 15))
 (segment (start 106.68 58.42) (end 106.68 61.248428) (width 1) (layer "F.Cu") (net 15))
 (via (at 88.9 78.74) (size 2) (drill 1.1) (layers "F.Cu" "B.Cu") (free) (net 15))
 (segment (start 88.9 78.74) (end 88.9 91.44) (width 1) (layer "B.Cu") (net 15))
 (segment (start 86.36 77.47) (end 86.36 83.82) (width 1) (layer "F.Cu") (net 16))
 (segment (start 104.14 59.69) (end 86.36 77.47) (width 1) (layer "F.Cu") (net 16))
 (segment (start 104.14 58.42) (end 104.14 59.69) (width 1) (layer "F.Cu") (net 16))
 (via (at 86.36 83.82) (size 2) (drill 1.1) (layers "F.Cu" "B.Cu") (free) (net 16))
 (segment (start 86.36 83.82) (end 86.36 91.44) (width 1) (layer "B.Cu") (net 16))
 (segment (start 124.46 58.42) (end 124.46 83.82) (width 1) (layer "F.Cu") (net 17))
 (via (at 124.46 83.82) (size 2) (drill 1.1) (layers "F.Cu" "B.Cu") (free) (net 17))
 (segment (start 124.46 83.82) (end 124.46 91.44) (width 1) (layer "B.Cu") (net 17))
 (segment (start 132.08 60.96) (end 160.02 88.9) (width 1) (layer "F.Cu") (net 25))
 (segment (start 160.02 98.08) (end 156.495 101.605) (width 1) (layer "F.Cu") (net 25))
 (segment (start 156.495 101.605) (end 155.645 101.605) (width 1) (layer "F.Cu") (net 25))
 (segment (start 132.08 58.42) (end 132.08 60.96) (width 1) (layer "F.Cu") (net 25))
 (segment (start 160.02 88.9) (end 160.02 98.08) (width 1) (layer "F.Cu") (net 25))
 (segment (start 129.54 58.42) (end 129.54 62.23) (width 1) (layer "F.Cu") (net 26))
 (segment (start 154.795 104.145) (end 155.645 104.145) (width 1) (layer "F.Cu") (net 26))
 (segment (start 152.4 101.75) (end 154.795 104.145) (width 1) (layer "F.Cu") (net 26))
 (segment (start 129.54 62.23) (end 152.4 85.09) (width 1) (layer "F.Cu") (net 26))
 (segment (start 152.4 85.09) (end 152.4 101.75) (width 1) (layer "F.Cu") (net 26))
 (segment (start 150.4 102.578428) (end 154.506572 106.685) (width 1) (layer "F.Cu") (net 27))
 (segment (start 127 58.42) (end 127 63.788428) (width 1) (layer "F.Cu") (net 27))
 (segment (start 127 63.788428) (end 150.4 87.188428) (width 1) (layer "F.Cu") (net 27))
 (segment (start 154.506572 106.685) (end 155.645 106.685) (width 1) (layer "F.Cu") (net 27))
 (segment (start 150.4 87.188428) (end 150.4 102.578428) (width 1) (layer "F.Cu") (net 27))
 (segment (start 114.28868 54.61) (end 146.05 54.61) (width 1) (layer "F.Cu") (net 3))
 (segment (start 111.76 57.13868) (end 114.28868 54.61) (width 1) (layer "F.Cu") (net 3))
 (segment (start 152.4 60.96) (end 165.1 60.96) (width 1) (layer "F.Cu") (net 3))
 (segment (start 111.76 58.42) (end 111.76 57.13868) (width 1) (layer "F.Cu") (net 3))
 (segment (start 146.05 54.61) (end 152.4 60.96) (width 1) (layer "F.Cu") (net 3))
 (segment (start 139.585 105.464185) (end 138.369185 106.68) (width 1) (layer "F.Cu") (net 24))
 (segment (start 141.194194 103.854991) (end 141.145824 103.854991) (width 1) (layer "F.Cu") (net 24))
 (segment (start 147.425 95.415815) (end 147.425 97.624185) (width 1) (layer "F.Cu") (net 24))
 (segment (start 130.52 98.08) (end 134.745009 93.854991) (width 1) (layer "F.Cu") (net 24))
 (segment (start 134.745009 93.854991) (end 145.864176 93.854991) (width 1) (layer "F.Cu") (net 24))
 (segment (start 141.145824 103.854991) (end 139.585 105.415815) (width 1) (layer "F.Cu") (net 24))
 (segment (start 147.425 97.624185) (end 141.194194 103.854991) (width 1) (layer "F.Cu") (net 24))
 (segment (start 139.585 105.415815) (end 139.585 105.464185) (width 1) (layer "F.Cu") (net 24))
 (segment (start 138.369185 106.68) (end 137.16 106.68) (width 1) (layer "F.Cu") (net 24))
 (segment (start 145.864176 93.854991) (end 147.425 95.415815) (width 1) (layer "F.Cu") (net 24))
 (segment (start 114.86 98.08) (end 130.52 98.08) (width 1) (layer "F.Cu") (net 24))
 (segment (start 127 106.68) (end 127 105.898244) (width 1) (layer "F.Cu") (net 28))
 (segment (start 127 105.898244) (end 136.378244 96.52) (width 1) (layer "F.Cu") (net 28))
 (segment (start 136.378244 96.52) (end 144.755 96.52) (width 1) (layer "F.Cu") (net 28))
 (segment (start 127 101.6) (end 124.46 104.14) (width 1) (layer "F.Cu") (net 21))
 (segment (start 124.46 104.14) (end 124.46 106.68) (width 1) (layer "F.Cu") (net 21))
 (segment (start 92.511 95.504) (end 127 95.504) (width 1) (layer "F.Cu") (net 21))
 (segment (start 91.415 96.6) (end 92.511 95.504) (width 1) (layer "F.Cu") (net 21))
 (via (at 127 95.504) (size 2) (drill 1.1) (layers "F.Cu" "B.Cu") (free) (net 21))
 (via (at 127 101.6) (size 2) (drill 1.1) (layers "F.Cu" "B.Cu") (free) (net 21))
 (segment (start 127 101.6) (end 127 95.504) (width 1) (layer "B.Cu") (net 21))
 (segment (start 190.4125 88.8125) (end 180.34 78.74) (width 1) (layer "B.Cu") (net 18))
 (segment (start 172.72 86.36) (end 180.34 78.74) (width 1) (layer "B.Cu") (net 18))
 (segment (start 167.72 86.36) (end 172.72 86.36) (width 1) (layer "B.Cu") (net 18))
 (segment (start 193.04 83.82) (end 195.54 83.82) (width 1) (layer "B.Cu") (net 18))
 (segment (start 195.54 83.82) (end 195.54 85.321224) (width 1) (layer "B.Cu") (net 18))
 (segment (start 185.42 68.58) (end 195.54 78.7) (width 1) (layer "B.Cu") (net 18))
 (segment (start 195.538777 85.322447) (end 195.538777 87.37665) (width 1) (layer "B.Cu") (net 18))
 (segment (start 194.102927 88.8125) (end 190.4125 88.8125) (width 1) (layer "B.Cu") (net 18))
 (segment (start 195.54 85.321224) (end 195.538777 85.322447) (width 1) (layer "B.Cu") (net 18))
 (segment (start 195.538777 87.37665) (end 194.102927 88.8125) (width 1) (layer "B.Cu") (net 18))
 (segment (start 195.54 78.7) (end 195.54 83.82) (width 1) (layer "B.Cu") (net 18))
 (segment (start 175.74 71.12) (end 177.8 71.12) (width 1) (layer "B.Cu") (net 19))
 (segment (start 172.72 60.96) (end 172.72 68.1) (width 1) (layer "B.Cu") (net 19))
 (segment (start 182.72 77.316567) (end 182.72 76.04) (width 1) (layer "B.Cu") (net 19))
 (segment (start 190.5 85.09) (end 190.493433 85.09) (width 1) (layer "B.Cu") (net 19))
 (segment (start 193.04 86.36) (end 191.77 86.36) (width 1) (layer "B.Cu") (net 19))
 (segment (start 172.72 68.1) (end 175.74 71.12) (width 1) (layer "B.Cu") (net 19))
 (segment (start 190.493433 85.09) (end 182.72 77.316567) (width 1) (layer "B.Cu") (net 19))
 (segment (start 167.64 55.88) (end 172.72 60.96) (width 1) (layer "B.Cu") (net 19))
 (segment (start 182.72 76.04) (end 177.8 71.12) (width 1) (layer "B.Cu") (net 19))
 (segment (start 191.77 86.36) (end 190.5 85.09) (width 1) (layer "B.Cu") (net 19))
 (segment (start 162.56 55.88) (end 167.64 55.88) (width 1) (layer "B.Cu") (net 19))
 (segment (start 169.474422 68.58) (end 170.18 68.58) (width 1) (layer "B.Cu") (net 4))
 (segment (start 165.1 72.954422) (end 169.474422 68.58) (width 1) (layer "B.Cu") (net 4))
 (segment (start 165.1 73.66) (end 165.1 72.954422) (width 1) (layer "B.Cu") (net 4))
 (segment (start 175.26 73.66) (end 175.26 67.78) (width 1) (layer "F.Cu") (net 20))
 (segment (start 177 66.04) (end 177.8 66.04) (width 1) (layer "F.Cu") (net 20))
 (segment (start 170.18 78.74) (end 175.26 73.66) (width 1) (layer "F.Cu") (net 20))
 (segment (start 175.26 67.78) (end 177 66.04) (width 1) (layer "F.Cu") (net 20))
 (segment (start 165.1 78.74) (end 170.18 78.74) (width 1) (layer "F.Cu") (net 20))
 (segment (start 193.04 81.28) (end 190.5 81.28) (width 1) (layer "B.Cu") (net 2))
 (segment (start 180.34 55.88) (end 185.42 60.96) (width 1) (layer "B.Cu") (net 2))
 (segment (start 185.42 75.005119) (end 185.42 76.2) (width 1) (layer "B.Cu") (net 2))
 (segment (start 190.5 81.28) (end 185.42 76.2) (width 1) (layer "B.Cu") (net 2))
 (segment (start 177.8 55.88) (end 180.34 55.88) (width 1) (layer "B.Cu") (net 2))
 (segment (start 182.645 72.230119) (end 185.42 75.005119) (width 1) (layer "B.Cu") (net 2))
 (segment (start 185.42 60.96) (end 182.645 63.735) (width 1) (layer "B.Cu") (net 2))
 (segment (start 182.645 63.735) (end 182.645 72.230119) (width 1) (layer "B.Cu") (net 2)))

